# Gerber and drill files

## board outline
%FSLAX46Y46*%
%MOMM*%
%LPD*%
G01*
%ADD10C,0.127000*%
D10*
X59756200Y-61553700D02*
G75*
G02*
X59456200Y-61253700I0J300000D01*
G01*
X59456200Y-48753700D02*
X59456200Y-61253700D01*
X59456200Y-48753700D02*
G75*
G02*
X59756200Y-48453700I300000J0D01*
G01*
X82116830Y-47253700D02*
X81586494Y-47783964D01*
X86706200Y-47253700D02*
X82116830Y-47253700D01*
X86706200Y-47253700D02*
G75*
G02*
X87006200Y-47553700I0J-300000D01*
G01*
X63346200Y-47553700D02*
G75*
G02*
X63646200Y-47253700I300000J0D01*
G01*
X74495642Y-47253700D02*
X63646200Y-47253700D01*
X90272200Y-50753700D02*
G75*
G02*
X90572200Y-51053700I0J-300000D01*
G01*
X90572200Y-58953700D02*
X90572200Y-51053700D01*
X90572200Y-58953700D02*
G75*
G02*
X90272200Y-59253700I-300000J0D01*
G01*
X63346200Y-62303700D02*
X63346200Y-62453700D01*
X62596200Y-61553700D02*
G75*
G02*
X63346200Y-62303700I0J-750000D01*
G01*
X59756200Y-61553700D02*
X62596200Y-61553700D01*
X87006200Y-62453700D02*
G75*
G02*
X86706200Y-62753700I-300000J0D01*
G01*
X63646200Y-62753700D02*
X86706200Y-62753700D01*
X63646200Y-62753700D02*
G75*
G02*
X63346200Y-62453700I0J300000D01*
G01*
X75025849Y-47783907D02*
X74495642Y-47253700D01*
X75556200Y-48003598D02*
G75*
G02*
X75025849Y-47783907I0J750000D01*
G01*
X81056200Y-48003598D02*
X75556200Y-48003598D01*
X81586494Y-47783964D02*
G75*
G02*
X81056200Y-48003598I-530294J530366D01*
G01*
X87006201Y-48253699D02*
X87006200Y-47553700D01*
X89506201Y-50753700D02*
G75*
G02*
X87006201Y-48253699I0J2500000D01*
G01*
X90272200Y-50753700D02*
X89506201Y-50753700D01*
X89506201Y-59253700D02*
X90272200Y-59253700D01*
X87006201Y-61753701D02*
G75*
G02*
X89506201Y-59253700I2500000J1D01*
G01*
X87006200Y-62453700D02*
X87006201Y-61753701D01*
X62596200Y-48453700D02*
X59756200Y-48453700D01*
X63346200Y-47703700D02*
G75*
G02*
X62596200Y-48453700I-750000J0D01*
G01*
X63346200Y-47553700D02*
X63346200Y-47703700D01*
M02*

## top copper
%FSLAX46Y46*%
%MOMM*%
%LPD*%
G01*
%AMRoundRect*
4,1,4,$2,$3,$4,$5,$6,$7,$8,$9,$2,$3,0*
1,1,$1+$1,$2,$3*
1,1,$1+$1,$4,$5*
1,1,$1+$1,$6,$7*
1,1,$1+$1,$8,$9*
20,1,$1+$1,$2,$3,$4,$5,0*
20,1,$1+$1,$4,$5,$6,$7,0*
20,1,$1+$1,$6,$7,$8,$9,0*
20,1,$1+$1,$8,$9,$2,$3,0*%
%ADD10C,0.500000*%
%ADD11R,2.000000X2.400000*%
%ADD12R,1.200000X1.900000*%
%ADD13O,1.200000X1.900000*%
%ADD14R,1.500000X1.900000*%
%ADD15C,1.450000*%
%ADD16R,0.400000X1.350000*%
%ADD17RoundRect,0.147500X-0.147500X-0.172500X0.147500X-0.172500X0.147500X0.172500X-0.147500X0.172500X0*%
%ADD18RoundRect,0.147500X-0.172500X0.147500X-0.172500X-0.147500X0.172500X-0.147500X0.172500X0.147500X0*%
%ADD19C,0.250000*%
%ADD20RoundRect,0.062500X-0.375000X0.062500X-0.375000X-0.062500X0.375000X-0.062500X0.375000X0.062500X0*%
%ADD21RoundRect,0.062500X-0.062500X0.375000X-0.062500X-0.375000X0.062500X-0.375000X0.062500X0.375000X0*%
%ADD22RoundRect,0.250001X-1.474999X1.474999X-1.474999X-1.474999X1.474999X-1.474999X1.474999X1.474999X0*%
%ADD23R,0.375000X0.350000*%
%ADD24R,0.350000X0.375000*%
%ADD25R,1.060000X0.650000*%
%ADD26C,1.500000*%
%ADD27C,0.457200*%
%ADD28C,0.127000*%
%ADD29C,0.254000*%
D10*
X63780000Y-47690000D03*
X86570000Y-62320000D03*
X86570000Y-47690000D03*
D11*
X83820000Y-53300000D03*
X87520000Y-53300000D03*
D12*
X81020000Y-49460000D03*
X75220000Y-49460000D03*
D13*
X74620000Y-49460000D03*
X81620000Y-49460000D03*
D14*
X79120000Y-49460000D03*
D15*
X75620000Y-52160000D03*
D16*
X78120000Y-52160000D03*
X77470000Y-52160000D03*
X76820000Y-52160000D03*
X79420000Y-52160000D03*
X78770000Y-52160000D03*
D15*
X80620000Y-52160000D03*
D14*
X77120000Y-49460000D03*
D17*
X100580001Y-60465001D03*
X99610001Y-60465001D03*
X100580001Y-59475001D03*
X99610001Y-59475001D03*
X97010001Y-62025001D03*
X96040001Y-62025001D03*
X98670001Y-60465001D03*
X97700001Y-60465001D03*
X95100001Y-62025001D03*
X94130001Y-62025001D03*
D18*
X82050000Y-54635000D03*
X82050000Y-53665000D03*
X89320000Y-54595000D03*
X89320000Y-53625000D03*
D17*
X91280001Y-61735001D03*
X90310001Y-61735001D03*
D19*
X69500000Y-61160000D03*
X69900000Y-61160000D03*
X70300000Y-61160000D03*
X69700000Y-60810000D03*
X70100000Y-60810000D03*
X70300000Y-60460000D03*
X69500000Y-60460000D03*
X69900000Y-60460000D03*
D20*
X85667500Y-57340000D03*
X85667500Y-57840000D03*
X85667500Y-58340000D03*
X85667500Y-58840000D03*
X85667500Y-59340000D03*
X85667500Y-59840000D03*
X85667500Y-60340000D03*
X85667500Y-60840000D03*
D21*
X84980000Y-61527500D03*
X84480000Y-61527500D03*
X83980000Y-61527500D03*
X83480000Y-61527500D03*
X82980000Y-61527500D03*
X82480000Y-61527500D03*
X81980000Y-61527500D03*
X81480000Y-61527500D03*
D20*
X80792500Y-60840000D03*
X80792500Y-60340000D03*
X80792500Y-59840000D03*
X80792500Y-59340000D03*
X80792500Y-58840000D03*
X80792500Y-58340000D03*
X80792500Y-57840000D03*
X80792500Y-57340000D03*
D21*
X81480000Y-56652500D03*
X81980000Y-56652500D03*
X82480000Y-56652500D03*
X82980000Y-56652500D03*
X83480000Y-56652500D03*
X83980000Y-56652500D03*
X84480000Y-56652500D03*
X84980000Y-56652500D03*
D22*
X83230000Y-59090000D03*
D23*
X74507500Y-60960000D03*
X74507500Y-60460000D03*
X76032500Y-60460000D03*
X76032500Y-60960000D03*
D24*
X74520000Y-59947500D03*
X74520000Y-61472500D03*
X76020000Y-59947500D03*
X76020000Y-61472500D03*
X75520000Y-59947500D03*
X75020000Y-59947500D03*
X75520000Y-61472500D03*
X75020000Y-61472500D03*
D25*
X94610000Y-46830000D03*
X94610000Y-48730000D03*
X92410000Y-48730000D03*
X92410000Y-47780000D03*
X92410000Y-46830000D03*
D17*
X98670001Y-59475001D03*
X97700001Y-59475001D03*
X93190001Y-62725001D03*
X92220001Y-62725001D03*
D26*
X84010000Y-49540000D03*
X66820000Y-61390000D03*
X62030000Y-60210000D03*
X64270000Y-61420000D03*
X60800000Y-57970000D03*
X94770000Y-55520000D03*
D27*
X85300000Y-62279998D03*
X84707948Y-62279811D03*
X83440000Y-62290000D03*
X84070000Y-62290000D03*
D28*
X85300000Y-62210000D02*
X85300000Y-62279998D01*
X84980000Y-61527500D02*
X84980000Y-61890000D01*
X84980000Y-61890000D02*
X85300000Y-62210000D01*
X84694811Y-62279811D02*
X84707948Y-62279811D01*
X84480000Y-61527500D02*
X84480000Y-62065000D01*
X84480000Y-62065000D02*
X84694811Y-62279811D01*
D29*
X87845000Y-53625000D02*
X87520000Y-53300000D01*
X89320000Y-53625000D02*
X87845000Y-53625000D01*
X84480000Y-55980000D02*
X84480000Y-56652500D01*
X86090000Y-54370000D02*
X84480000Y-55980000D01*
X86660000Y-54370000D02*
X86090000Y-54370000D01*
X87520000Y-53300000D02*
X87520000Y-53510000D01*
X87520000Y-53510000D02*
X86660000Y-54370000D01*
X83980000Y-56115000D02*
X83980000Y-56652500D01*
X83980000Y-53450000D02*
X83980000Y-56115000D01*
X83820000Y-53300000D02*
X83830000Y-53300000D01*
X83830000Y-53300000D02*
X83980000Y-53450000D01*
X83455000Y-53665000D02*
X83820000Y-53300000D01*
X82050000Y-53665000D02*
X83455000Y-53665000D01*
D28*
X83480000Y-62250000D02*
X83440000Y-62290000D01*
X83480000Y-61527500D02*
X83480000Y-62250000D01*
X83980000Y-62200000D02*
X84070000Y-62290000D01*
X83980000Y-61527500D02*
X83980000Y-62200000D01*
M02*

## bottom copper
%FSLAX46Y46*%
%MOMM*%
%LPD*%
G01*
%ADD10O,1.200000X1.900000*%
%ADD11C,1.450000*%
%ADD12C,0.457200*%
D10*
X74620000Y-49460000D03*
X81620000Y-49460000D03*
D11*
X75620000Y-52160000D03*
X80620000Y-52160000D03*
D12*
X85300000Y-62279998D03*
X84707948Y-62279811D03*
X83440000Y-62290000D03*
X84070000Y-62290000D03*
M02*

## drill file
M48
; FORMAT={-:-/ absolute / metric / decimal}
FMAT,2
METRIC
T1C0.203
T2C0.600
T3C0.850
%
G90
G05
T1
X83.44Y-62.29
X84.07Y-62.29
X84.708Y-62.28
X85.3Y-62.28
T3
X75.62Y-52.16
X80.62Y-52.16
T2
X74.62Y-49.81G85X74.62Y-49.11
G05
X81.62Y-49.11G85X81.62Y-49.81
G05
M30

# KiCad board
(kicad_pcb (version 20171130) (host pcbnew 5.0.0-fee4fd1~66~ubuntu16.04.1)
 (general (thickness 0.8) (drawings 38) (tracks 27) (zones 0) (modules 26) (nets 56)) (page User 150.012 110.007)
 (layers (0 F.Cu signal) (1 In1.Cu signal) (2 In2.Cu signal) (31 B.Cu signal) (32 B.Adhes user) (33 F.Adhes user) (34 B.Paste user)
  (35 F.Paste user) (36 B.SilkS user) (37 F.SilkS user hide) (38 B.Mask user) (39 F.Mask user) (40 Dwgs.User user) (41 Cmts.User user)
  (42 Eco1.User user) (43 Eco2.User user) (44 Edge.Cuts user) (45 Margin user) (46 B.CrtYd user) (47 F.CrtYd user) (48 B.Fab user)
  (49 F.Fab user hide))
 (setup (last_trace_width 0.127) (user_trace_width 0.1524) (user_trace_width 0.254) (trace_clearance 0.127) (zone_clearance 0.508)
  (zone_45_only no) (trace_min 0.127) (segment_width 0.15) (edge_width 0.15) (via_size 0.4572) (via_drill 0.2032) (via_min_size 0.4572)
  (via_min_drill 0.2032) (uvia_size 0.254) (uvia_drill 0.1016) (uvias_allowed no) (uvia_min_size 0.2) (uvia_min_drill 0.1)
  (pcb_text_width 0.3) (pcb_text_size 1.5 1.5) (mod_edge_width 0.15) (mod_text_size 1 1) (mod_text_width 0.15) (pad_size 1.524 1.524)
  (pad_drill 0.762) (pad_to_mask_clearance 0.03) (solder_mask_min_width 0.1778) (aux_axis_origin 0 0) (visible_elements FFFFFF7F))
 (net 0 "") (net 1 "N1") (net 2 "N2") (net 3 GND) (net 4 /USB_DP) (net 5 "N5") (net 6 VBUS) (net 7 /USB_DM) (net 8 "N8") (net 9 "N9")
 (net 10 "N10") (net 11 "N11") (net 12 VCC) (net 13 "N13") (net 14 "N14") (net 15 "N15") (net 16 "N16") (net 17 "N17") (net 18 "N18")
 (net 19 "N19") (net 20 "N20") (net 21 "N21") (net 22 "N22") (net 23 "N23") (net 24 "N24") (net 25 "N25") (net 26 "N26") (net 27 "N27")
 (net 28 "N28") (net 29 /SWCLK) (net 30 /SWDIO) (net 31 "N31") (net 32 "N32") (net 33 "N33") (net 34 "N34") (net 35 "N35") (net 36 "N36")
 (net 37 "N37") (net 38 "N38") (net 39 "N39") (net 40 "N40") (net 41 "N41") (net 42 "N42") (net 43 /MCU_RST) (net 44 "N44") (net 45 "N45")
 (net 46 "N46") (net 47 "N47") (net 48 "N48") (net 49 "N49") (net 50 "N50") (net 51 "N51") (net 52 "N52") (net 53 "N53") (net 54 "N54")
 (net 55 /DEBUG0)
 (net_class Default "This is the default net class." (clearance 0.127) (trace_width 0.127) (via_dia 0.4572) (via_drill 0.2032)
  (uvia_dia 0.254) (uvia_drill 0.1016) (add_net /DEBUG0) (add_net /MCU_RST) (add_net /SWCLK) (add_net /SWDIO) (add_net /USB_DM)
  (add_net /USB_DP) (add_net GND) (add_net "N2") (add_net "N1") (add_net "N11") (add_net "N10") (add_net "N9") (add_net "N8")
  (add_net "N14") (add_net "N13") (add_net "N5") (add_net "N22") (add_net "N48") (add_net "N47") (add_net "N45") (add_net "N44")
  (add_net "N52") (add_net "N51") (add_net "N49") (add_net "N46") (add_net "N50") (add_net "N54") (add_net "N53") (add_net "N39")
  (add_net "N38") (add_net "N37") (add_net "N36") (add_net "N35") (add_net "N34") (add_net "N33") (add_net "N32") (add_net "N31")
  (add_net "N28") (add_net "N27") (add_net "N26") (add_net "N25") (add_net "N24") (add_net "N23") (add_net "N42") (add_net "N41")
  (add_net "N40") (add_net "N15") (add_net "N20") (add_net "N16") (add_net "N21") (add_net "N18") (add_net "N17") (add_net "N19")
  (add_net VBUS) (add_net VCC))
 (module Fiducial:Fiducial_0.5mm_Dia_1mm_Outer (layer F.Cu) (at 63.78 47.69)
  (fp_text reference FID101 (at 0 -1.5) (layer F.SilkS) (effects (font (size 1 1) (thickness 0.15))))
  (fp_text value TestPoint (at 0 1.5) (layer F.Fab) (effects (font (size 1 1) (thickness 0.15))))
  (pad ~ smd circle (at 0 0) (size 0.5 0.5) (layers F.Cu F.Mask) (solder_mask_margin 0.25) (clearance 0.25)))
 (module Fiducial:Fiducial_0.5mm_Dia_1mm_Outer (layer F.Cu) (at 86.57 62.32)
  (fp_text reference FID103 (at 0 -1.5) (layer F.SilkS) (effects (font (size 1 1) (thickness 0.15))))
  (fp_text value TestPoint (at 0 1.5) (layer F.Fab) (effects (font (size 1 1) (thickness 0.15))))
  (pad ~ smd circle (at 0 0) (size 0.5 0.5) (layers F.Cu F.Mask) (solder_mask_margin 0.25) (clearance 0.25)))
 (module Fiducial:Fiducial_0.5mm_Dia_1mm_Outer (layer F.Cu) (at 86.57 47.69)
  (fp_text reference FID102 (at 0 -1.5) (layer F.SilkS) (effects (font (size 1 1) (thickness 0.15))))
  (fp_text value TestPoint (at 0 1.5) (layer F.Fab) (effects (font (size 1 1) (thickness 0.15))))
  (pad ~ smd circle (at 0 0) (size 0.5 0.5) (layers F.Cu F.Mask) (solder_mask_margin 0.25) (clearance 0.25)))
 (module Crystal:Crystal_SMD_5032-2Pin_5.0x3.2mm (layer F.Cu) (at 85.67 53.3 180)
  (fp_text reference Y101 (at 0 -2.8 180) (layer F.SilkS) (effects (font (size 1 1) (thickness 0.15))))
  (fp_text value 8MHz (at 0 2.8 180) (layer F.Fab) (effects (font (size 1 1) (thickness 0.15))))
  (pad 2 smd rect (at 1.85 0 180) (size 2 2.4) (layers F.Cu F.Paste F.Mask) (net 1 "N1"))
  (pad 1 smd rect (at -1.85 0 180) (size 2 2.4) (layers F.Cu F.Paste F.Mask) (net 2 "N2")))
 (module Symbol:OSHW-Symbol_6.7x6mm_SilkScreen (layer F.Cu) (at 67.84 53.39 270)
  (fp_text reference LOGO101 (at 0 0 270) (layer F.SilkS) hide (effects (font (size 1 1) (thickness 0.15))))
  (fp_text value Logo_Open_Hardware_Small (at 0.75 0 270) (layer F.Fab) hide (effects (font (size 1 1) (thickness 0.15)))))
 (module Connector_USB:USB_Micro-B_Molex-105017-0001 (layer F.Cu) (at 78.12 50.6975 180)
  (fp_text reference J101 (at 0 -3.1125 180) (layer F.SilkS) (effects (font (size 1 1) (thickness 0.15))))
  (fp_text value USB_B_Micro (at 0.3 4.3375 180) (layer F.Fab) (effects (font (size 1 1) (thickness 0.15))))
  (pad 6 smd rect (at -2.9 1.2375 180) (size 1.2 1.9) (layers F.Cu F.Mask) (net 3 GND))
  (pad 6 smd rect (at 2.9 1.2375 180) (size 1.2 1.9) (layers F.Cu F.Mask) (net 3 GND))
  (pad 6 thru_hole oval (at 3.5 1.2375 180) (size 1.2 1.9) (drill oval 0.6 1.3) (layers *.Cu *.Mask) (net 3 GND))
  (pad 6 thru_hole oval (at -3.5 1.2375) (size 1.2 1.9) (drill oval 0.6 1.3) (layers *.Cu *.Mask) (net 3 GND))
  (pad 6 smd rect (at -1 1.2375 180) (size 1.5 1.9) (layers F.Cu F.Paste F.Mask) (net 3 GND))
  (pad 6 thru_hole circle (at 2.5 -1.4625 180) (size 1.45 1.45) (drill 0.85) (layers *.Cu *.Mask) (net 3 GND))
  (pad 3 smd rect (at 0 -1.4625 180) (size 0.4 1.35) (layers F.Cu F.Paste F.Mask) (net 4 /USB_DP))
  (pad 4 smd rect (at 0.65 -1.4625 180) (size 0.4 1.35) (layers F.Cu F.Paste F.Mask) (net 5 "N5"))
  (pad 5 smd rect (at 1.3 -1.4625 180) (size 0.4 1.35) (layers F.Cu F.Paste F.Mask) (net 3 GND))
  (pad 1 smd rect (at -1.3 -1.4625 180) (size 0.4 1.35) (layers F.Cu F.Paste F.Mask) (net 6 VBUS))
  (pad 2 smd rect (at -0.65 -1.4625 180) (size 0.4 1.35) (layers F.Cu F.Paste F.Mask) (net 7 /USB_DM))
  (pad 6 thru_hole circle (at -2.5 -1.4625 180) (size 1.45 1.45) (drill 0.85) (layers *.Cu *.Mask) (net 3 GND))
  (pad 6 smd rect (at 1 1.2375 180) (size 1.5 1.9) (layers F.Cu F.Paste F.Mask) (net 3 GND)))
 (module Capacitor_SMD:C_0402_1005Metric (layer F.Cu) (at 100.095001 60.465001)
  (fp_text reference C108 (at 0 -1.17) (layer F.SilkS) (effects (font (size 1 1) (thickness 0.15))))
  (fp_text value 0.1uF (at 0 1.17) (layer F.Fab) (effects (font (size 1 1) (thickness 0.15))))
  (pad 2 smd roundrect (at 0.485 0) (size 0.59 0.64) (layers F.Cu F.Paste F.Mask) (roundrect_rratio 0.25) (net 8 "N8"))
  (pad 1 smd roundrect (at -0.485 0) (size 0.59 0.64) (layers F.Cu F.Paste F.Mask) (roundrect_rratio 0.25) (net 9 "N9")))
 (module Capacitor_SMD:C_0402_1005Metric (layer F.Cu) (at 100.095001 59.475001)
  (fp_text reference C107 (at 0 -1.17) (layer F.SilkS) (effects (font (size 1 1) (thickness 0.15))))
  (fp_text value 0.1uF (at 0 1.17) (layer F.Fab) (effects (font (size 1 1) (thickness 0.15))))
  (pad 2 smd roundrect (at 0.485 0) (size 0.59 0.64) (layers F.Cu F.Paste F.Mask) (roundrect_rratio 0.25) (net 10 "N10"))
  (pad 1 smd roundrect (at -0.485 0) (size 0.59 0.64) (layers F.Cu F.Paste F.Mask) (roundrect_rratio 0.25) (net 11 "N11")))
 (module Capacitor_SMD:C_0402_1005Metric (layer F.Cu) (at 96.525001 62.025001)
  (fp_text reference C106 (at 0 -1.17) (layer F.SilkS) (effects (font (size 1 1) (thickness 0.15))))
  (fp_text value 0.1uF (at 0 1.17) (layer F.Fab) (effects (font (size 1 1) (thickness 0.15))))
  (pad 2 smd roundrect (at 0.485 0) (size 0.59 0.64) (layers F.Cu F.Paste F.Mask) (roundrect_rratio 0.25) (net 3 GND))
  (pad 1 smd roundrect (at -0.485 0) (size 0.59 0.64) (layers F.Cu F.Paste F.Mask) (roundrect_rratio 0.25) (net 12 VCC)))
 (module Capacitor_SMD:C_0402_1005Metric (layer F.Cu) (at 98.185001 60.465001)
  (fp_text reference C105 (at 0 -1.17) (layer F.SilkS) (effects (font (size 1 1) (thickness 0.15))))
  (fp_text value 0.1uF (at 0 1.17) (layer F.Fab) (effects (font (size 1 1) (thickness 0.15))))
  (pad 2 smd roundrect (at 0.485 0) (size 0.59 0.64) (layers F.Cu F.Paste F.Mask) (roundrect_rratio 0.25) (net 3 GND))
  (pad 1 smd roundrect (at -0.485 0) (size 0.59 0.64) (layers F.Cu F.Paste F.Mask) (roundrect_rratio 0.25) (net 12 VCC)))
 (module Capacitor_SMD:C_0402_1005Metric (layer F.Cu) (at 94.615001 62.025001)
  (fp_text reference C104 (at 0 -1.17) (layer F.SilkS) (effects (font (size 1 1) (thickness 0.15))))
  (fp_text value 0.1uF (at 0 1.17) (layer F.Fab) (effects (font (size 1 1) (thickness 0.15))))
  (pad 2 smd roundrect (at 0.485 0) (size 0.59 0.64) (layers F.Cu F.Paste F.Mask) (roundrect_rratio 0.25) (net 3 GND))
  (pad 1 smd roundrect (at -0.485 0) (size 0.59 0.64) (layers F.Cu F.Paste F.Mask) (roundrect_rratio 0.25) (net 12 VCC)))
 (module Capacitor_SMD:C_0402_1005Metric (layer F.Cu) (at 82.05 54.15 270)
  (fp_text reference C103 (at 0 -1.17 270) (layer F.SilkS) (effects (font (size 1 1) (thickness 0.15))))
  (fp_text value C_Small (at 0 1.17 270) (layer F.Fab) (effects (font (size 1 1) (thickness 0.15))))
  (pad 2 smd roundrect (at 0.485 0 270) (size 0.59 0.64) (layers F.Cu F.Paste F.Mask) (roundrect_rratio 0.25) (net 3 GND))
  (pad 1 smd roundrect (at -0.485 0 270) (size 0.59 0.64) (layers F.Cu F.Paste F.Mask) (roundrect_rratio 0.25) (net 1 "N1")))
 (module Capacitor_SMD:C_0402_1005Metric (layer F.Cu) (at 89.32 54.11 270)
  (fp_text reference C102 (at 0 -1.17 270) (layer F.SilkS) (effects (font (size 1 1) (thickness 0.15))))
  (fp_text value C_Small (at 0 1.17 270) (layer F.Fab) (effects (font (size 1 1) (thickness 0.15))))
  (pad 2 smd roundrect (at 0.485 0 270) (size 0.59 0.64) (layers F.Cu F.Paste F.Mask) (roundrect_rratio 0.25) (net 3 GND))
  (pad 1 smd roundrect (at -0.485 0 270) (size 0.59 0.64) (layers F.Cu F.Paste F.Mask) (roundrect_rratio 0.25) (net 2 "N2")))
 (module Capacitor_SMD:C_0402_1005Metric (layer F.Cu) (at 90.795001 61.735001)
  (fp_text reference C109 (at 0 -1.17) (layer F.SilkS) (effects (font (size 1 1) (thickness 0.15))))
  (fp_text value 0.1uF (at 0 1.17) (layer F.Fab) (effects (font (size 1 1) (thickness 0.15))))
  (pad 2 smd roundrect (at 0.485 0) (size 0.59 0.64) (layers F.Cu F.Paste F.Mask) (roundrect_rratio 0.25) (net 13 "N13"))
  (pad 1 smd roundrect (at -0.485 0) (size 0.59 0.64) (layers F.Cu F.Paste F.Mask) (roundrect_rratio 0.25) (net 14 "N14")))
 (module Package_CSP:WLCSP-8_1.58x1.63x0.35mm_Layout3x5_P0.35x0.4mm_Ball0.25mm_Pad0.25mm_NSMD (layer F.Cu) (at 69.9 60.81 90)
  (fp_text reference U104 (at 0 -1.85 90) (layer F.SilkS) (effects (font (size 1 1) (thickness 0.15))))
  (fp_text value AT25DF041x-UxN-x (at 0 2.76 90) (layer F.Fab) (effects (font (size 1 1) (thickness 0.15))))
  (pad A1 smd circle (at -0.35 -0.4 90) (size 0.25 0.25) (layers F.Cu F.Paste F.Mask) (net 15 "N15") (solder_mask_margin 0.03))
  (pad C1 smd circle (at -0.35 0 90) (size 0.25 0.25) (layers F.Cu F.Paste F.Mask) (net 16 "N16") (solder_mask_margin 0.03))
  (pad E1 smd circle (at -0.35 0.4 90) (size 0.25 0.25) (layers F.Cu F.Paste F.Mask) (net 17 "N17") (solder_mask_margin 0.03))
  (pad B2 smd circle (at 0 -0.2 90) (size 0.25 0.25) (layers F.Cu F.Paste F.Mask) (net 3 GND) (solder_mask_margin 0.03))
  (pad D2 smd circle (at 0 0.2 90) (size 0.25 0.25) (layers F.Cu F.Paste F.Mask) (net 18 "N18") (solder_mask_margin 0.03))
  (pad E3 smd circle (at 0.35 0.4 90) (size 0.25 0.25) (layers F.Cu F.Paste F.Mask) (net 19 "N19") (solder_mask_margin 0.03))
  (pad A3 smd circle (at 0.35 -0.4 90) (size 0.25 0.25) (layers F.Cu F.Paste F.Mask) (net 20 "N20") (solder_mask_margin 0.03))
  (pad C3 smd circle (at 0.35 0 90) (size 0.25 0.25) (layers F.Cu F.Paste F.Mask) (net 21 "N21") (solder_mask_margin 0.03)))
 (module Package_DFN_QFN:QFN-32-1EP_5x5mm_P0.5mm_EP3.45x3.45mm (layer F.Cu) (at 83.23 59.09 270)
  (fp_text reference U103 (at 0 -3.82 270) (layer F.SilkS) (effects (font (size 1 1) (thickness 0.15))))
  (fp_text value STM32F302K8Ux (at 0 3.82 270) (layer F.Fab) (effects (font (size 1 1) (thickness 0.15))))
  (pad 32 smd roundrect (at -1.75 -2.4375 270) (size 0.25 0.875) (layers F.Cu F.Paste F.Mask) (roundrect_rratio 0.25) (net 3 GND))
  (pad 31 smd roundrect (at -1.25 -2.4375 270) (size 0.25 0.875) (layers F.Cu F.Paste F.Mask) (roundrect_rratio 0.25) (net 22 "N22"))
  (pad 30 smd roundrect (at -0.75 -2.4375 270) (size 0.25 0.875) (layers F.Cu F.Paste F.Mask) (roundrect_rratio 0.25) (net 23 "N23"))
  (pad 29 smd roundrect (at -0.25 -2.4375 270) (size 0.25 0.875) (layers F.Cu F.Paste F.Mask) (roundrect_rratio 0.25) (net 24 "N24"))
  (pad 28 smd roundrect (at 0.25 -2.4375 270) (size 0.25 0.875) (layers F.Cu F.Paste F.Mask) (roundrect_rratio 0.25) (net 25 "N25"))
  (pad 27 smd roundrect (at 0.75 -2.4375 270) (size 0.25 0.875) (layers F.Cu F.Paste F.Mask) (roundrect_rratio 0.25) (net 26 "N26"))
  (pad 26 smd roundrect (at 1.25 -2.4375 270) (size 0.25 0.875) (layers F.Cu F.Paste F.Mask) (roundrect_rratio 0.25) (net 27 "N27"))
  (pad 25 smd roundrect (at 1.75 -2.4375 270) (size 0.25 0.875) (layers F.Cu F.Paste F.Mask) (roundrect_rratio 0.25) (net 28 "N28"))
  (pad 24 smd roundrect (at 2.4375 -1.75 270) (size 0.875 0.25) (layers F.Cu F.Paste F.Mask) (roundrect_rratio 0.25) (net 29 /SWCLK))
  (pad 23 smd roundrect (at 2.4375 -1.25 270) (size 0.875 0.25) (layers F.Cu F.Paste F.Mask) (roundrect_rratio 0.25) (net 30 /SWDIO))
  (pad 22 smd roundrect (at 2.4375 -0.75 270) (size 0.875 0.25) (layers F.Cu F.Paste F.Mask) (roundrect_rratio 0.25) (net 4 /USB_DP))
  (pad 21 smd roundrect (at 2.4375 -0.25 270) (size 0.875 0.25) (layers F.Cu F.Paste F.Mask) (roundrect_rratio 0.25) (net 7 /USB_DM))
  (pad 20 smd roundrect (at 2.4375 0.25 270) (size 0.875 0.25) (layers F.Cu F.Paste F.Mask) (roundrect_rratio 0.25) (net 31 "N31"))
  (pad 19 smd roundrect (at 2.4375 0.75 270) (size 0.875 0.25) (layers F.Cu F.Paste F.Mask) (roundrect_rratio 0.25) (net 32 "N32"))
  (pad 18 smd roundrect (at 2.4375 1.25 270) (size 0.875 0.25) (layers F.Cu F.Paste F.Mask) (roundrect_rratio 0.25) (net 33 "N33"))
  (pad 17 smd roundrect (at 2.4375 1.75 270) (size 0.875 0.25) (layers F.Cu F.Paste F.Mask) (roundrect_rratio 0.25) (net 12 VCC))
  (pad 16 smd roundrect (at 1.75 2.4375 270) (size 0.25 0.875) (layers F.Cu F.Paste F.Mask) (roundrect_rratio 0.25) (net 3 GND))
  (pad 15 smd roundrect (at 1.25 2.4375 270) (size 0.25 0.875) (layers F.Cu F.Paste F.Mask) (roundrect_rratio 0.25) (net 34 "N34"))
  (pad 14 smd roundrect (at 0.75 2.4375 270) (size 0.25 0.875) (layers F.Cu F.Paste F.Mask) (roundrect_rratio 0.25) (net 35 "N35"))
  (pad 13 smd roundrect (at 0.25 2.4375 270) (size 0.25 0.875) (layers F.Cu F.Paste F.Mask) (roundrect_rratio 0.25) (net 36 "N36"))
  (pad 12 smd roundrect (at -0.25 2.4375 270) (size 0.25 0.875) (layers F.Cu F.Paste F.Mask) (roundrect_rratio 0.25) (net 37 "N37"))
  (pad 11 smd roundrect (at -0.75 2.4375 270) (size 0.25 0.875) (layers F.Cu F.Paste F.Mask) (roundrect_rratio 0.25) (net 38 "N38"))
  (pad 10 smd roundrect (at -1.25 2.4375 270) (size 0.25 0.875) (layers F.Cu F.Paste F.Mask) (roundrect_rratio 0.25) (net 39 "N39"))
  (pad 9 smd roundrect (at -1.75 2.4375 270) (size 0.25 0.875) (layers F.Cu F.Paste F.Mask) (roundrect_rratio 0.25) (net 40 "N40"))
  (pad 8 smd roundrect (at -2.4375 1.75 270) (size 0.875 0.25) (layers F.Cu F.Paste F.Mask) (roundrect_rratio 0.25) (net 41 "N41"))
  (pad 7 smd roundrect (at -2.4375 1.25 270) (size 0.875 0.25) (layers F.Cu F.Paste F.Mask) (roundrect_rratio 0.25) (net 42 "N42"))
  (pad 6 smd roundrect (at -2.4375 0.75 270) (size 0.875 0.25) (layers F.Cu F.Paste F.Mask) (roundrect_rratio 0.25) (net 3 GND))
  (pad 5 smd roundrect (at -2.4375 0.25 270) (size 0.875 0.25) (layers F.Cu F.Paste F.Mask) (roundrect_rratio 0.25) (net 12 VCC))
  (pad 4 smd roundrect (at -2.4375 -0.25 270) (size 0.875 0.25) (layers F.Cu F.Paste F.Mask) (roundrect_rratio 0.25) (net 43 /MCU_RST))
  (pad 3 smd roundrect (at -2.4375 -0.75 270) (size 0.875 0.25) (layers F.Cu F.Paste F.Mask) (roundrect_rratio 0.25) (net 1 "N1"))
  (pad 2 smd roundrect (at -2.4375 -1.25 270) (size 0.875 0.25) (layers F.Cu F.Paste F.Mask) (roundrect_rratio 0.25) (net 2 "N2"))
  (pad 1 smd roundrect (at -2.4375 -1.75 270) (size 0.875 0.25) (layers F.Cu F.Paste F.Mask) (roundrect_rratio 0.25) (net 12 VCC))
  (pad "" smd roundrect (at 1.15 1.15 270) (size 0.93 0.93) (layers F.Paste) (roundrect_rratio 0.25))
  (pad "" smd roundrect (at 1.15 0 270) (size 0.93 0.93) (layers F.Paste) (roundrect_rratio 0.25))
  (pad "" smd roundrect (at 1.15 -1.15 270) (size 0.93 0.93) (layers F.Paste) (roundrect_rratio 0.25))
  (pad "" smd roundrect (at 0 1.15 270) (size 0.93 0.93) (layers F.Paste) (roundrect_rratio 0.25))
  (pad "" smd roundrect (at 0 0 270) (size 0.93 0.93) (layers F.Paste) (roundrect_rratio 0.25))
  (pad "" smd roundrect (at 0 -1.15 270) (size 0.93 0.93) (layers F.Paste) (roundrect_rratio 0.25))
  (pad "" smd roundrect (at -1.15 1.15 270) (size 0.93 0.93) (layers F.Paste) (roundrect_rratio 0.25))
  (pad "" smd roundrect (at -1.15 0 270) (size 0.93 0.93) (layers F.Paste) (roundrect_rratio 0.25))
  (pad "" smd roundrect (at -1.15 -1.15 270) (size 0.93 0.93) (layers F.Paste) (roundrect_rratio 0.25))
  (pad 33 smd roundrect (at 0 0 270) (size 3.45 3.45) (layers F.Cu F.Mask) (roundrect_rratio 0.072464) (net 3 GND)))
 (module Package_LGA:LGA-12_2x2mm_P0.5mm (layer F.Cu) (at 75.27 60.71 90)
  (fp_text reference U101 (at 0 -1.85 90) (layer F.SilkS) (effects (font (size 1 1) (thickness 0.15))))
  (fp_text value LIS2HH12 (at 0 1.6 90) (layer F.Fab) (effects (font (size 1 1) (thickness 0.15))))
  (pad 12 smd rect (at -0.25 -0.7625 180) (size 0.375 0.35) (layers F.Cu F.Paste F.Mask) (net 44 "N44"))
  (pad 11 smd rect (at 0.25 -0.7625 180) (size 0.375 0.35) (layers F.Cu F.Paste F.Mask) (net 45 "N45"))
  (pad 6 smd rect (at 0.25 0.7625 180) (size 0.375 0.35) (layers F.Cu F.Paste F.Mask) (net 3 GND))
  (pad 5 smd rect (at -0.25 0.7625 180) (size 0.375 0.35) (layers F.Cu F.Paste F.Mask) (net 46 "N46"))
  (pad 10 smd rect (at 0.7625 -0.75 90) (size 0.375 0.35) (layers F.Cu F.Paste F.Mask) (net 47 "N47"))
  (pad 1 smd rect (at -0.7625 -0.75 90) (size 0.375 0.35) (layers F.Cu F.Paste F.Mask) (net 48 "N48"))
  (pad 7 smd rect (at 0.7625 0.75 90) (size 0.375 0.35) (layers F.Cu F.Paste F.Mask) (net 3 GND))
  (pad 4 smd rect (at -0.7625 0.75 90) (size 0.375 0.35) (layers F.Cu F.Paste F.Mask) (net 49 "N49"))
  (pad 8 smd rect (at 0.7625 0.25 90) (size 0.375 0.35) (layers F.Cu F.Paste F.Mask) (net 3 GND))
  (pad 9 smd rect (at 0.7625 -0.25 90) (size 0.375 0.35) (layers F.Cu F.Paste F.Mask) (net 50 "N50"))
  (pad 3 smd rect (at -0.7625 0.25 90) (size 0.375 0.35) (layers F.Cu F.Paste F.Mask) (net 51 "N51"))
  (pad 2 smd rect (at -0.7625 -0.25 90) (size 0.375 0.35) (layers F.Cu F.Paste F.Mask) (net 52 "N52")))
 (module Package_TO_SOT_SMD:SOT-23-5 (layer F.Cu) (at 93.51 47.78)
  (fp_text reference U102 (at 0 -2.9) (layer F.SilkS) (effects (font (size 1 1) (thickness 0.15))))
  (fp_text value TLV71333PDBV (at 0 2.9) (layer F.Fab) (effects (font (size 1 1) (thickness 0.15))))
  (pad 5 smd rect (at 1.1 -0.95) (size 1.06 0.65) (layers F.Cu F.Paste F.Mask) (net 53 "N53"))
  (pad 4 smd rect (at 1.1 0.95) (size 1.06 0.65) (layers F.Cu F.Paste F.Mask) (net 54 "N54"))
  (pad 3 smd rect (at -1.1 0.95) (size 1.06 0.65) (layers F.Cu F.Paste F.Mask) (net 6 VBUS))
  (pad 2 smd rect (at -1.1 0) (size 1.06 0.65) (layers F.Cu F.Paste F.Mask) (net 3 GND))
  (pad 1 smd rect (at -1.1 -0.95) (size 1.06 0.65) (layers F.Cu F.Paste F.Mask) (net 6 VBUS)))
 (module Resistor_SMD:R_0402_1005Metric (layer F.Cu) (at 98.185001 59.475001)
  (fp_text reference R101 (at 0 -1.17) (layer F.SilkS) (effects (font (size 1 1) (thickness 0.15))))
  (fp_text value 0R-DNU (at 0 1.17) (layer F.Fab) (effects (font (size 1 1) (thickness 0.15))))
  (pad 2 smd roundrect (at 0.485 0) (size 0.59 0.64) (layers F.Cu F.Paste F.Mask) (roundrect_rratio 0.25) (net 22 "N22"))
  (pad 1 smd roundrect (at -0.485 0) (size 0.59 0.64) (layers F.Cu F.Paste F.Mask) (roundrect_rratio 0.25) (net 12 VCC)))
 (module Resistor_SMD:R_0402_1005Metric (layer F.Cu) (at 92.705001 62.725001)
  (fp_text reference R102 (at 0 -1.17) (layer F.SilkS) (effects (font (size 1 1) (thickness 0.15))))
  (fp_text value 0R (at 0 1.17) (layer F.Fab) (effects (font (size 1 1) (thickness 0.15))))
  (pad 2 smd roundrect (at 0.485 0) (size 0.59 0.64) (layers F.Cu F.Paste F.Mask) (roundrect_rratio 0.25) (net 3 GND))
  (pad 1 smd roundrect (at -0.485 0) (size 0.59 0.64) (layers F.Cu F.Paste F.Mask) (roundrect_rratio 0.25) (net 22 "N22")))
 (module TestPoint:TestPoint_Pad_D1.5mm (layer F.Cu) (at 84.01 49.54)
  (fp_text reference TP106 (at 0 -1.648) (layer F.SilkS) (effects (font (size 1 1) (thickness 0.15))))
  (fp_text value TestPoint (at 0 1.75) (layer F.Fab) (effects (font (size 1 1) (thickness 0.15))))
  (pad 1 smd circle (at 0 0) (size 1.5 1.5) (layers F.Cu F.Mask) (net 3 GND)))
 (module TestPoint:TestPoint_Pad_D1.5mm (layer F.Cu) (at 66.82 61.39)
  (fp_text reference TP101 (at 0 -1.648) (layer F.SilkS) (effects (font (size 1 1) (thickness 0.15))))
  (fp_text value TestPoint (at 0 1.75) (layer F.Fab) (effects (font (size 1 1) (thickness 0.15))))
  (pad 1 smd circle (at 0 0) (size 1.5 1.5) (layers F.Cu F.Mask) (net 43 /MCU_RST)))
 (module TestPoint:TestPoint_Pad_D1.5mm (layer F.Cu) (at 62.03 60.21)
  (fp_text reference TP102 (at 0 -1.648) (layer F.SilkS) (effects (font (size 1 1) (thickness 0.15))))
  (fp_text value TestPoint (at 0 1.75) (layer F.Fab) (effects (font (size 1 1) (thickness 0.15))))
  (pad 1 smd circle (at 0 0) (size 1.5 1.5) (layers F.Cu F.Mask) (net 30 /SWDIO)))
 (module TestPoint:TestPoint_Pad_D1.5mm (layer F.Cu) (at 64.27 61.42)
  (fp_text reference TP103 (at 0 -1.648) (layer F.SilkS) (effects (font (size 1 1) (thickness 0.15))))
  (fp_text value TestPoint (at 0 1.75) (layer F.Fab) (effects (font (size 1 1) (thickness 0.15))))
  (pad 1 smd circle (at 0 0) (size 1.5 1.5) (layers F.Cu F.Mask) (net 29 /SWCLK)))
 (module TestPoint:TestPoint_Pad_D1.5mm (layer F.Cu) (at 60.8 57.97)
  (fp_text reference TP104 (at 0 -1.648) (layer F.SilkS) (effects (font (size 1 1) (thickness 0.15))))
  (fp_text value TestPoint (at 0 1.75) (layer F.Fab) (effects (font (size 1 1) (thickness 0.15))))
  (pad 1 smd circle (at 0 0) (size 1.5 1.5) (layers F.Cu F.Mask) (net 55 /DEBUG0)))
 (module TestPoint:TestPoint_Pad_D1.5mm (layer F.Cu) (at 94.77 55.52)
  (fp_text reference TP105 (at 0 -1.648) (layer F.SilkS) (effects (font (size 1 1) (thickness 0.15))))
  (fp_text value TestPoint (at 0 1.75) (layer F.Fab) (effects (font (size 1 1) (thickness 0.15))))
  (pad 1 smd circle (at 0 0) (size 1.5 1.5) (layers F.Cu F.Mask) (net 12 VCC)))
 (gr_arc (start 59.7562 61.2537) (end 59.4562 61.2537) (angle -90.00000085) (layer Edge.Cuts) (width 0.127))
 (gr_line (start 59.4562 48.7537) (end 59.4562 61.2537) (layer Edge.Cuts) (width 0.127))
 (gr_arc (start 59.7562 48.7537) (end 59.7562 48.4537) (angle -89.99999915) (layer Edge.Cuts) (width 0.127))
 (gr_line (start 82.11683 47.2537) (end 81.586494 47.783964) (layer Edge.Cuts) (width 0.127))
 (gr_line (start 86.7062 47.2537) (end 82.11683 47.2537) (layer Edge.Cuts) (width 0.127))
 (gr_arc (start 86.7062 47.5537) (end 87.0062 47.5537) (angle -90) (layer Edge.Cuts) (width 0.127))
 (gr_arc (start 63.6462 47.5537) (end 63.6462 47.2537) (angle -90) (layer Edge.Cuts) (width 0.127))
 (gr_line (start 74.495642 47.2537) (end 63.6462 47.2537) (layer Edge.Cuts) (width 0.127))
 (gr_arc (start 90.2722 51.0537) (end 90.5722 51.0537) (angle -90) (layer Edge.Cuts) (width 0.127))
 (gr_line (start 90.5722 58.9537) (end 90.5722 51.0537) (layer Edge.Cuts) (width 0.127))
 (gr_arc (start 90.2722 58.9537) (end 90.2722 59.2537) (angle -90) (layer Edge.Cuts) (width 0.127))
 (gr_line (start 63.3462 62.3037) (end 63.3462 62.4537) (layer Edge.Cuts) (width 0.127))
 (gr_arc (start 62.5962 62.3037) (end 63.3462 62.3037) (angle -90) (layer Edge.Cuts) (width 0.127))
 (gr_line (start 59.7562 61.5537) (end 62.5962 61.5537) (layer Edge.Cuts) (width 0.127))
 (gr_arc (start 86.7062 62.4537) (end 86.7062 62.7537) (angle -89.99999944) (layer Edge.Cuts) (width 0.127))
 (gr_line (start 63.6462 62.7537) (end 86.7062 62.7537) (layer Edge.Cuts) (width 0.127))
 (gr_arc (start 63.6462 62.4537) (end 63.3462 62.4537) (angle -90.00000056) (layer Edge.Cuts) (width 0.127))
 (gr_line (start 75.025849 47.783907) (end 74.495642 47.2537) (layer Edge.Cuts) (width 0.127))
 (gr_arc (start 75.5562 47.253598) (end 75.025849 47.783907) (angle -45.00225503) (layer Edge.Cuts) (width 0.127))
 (gr_line (start 81.0562 48.003598) (end 75.5562 48.003598) (layer Edge.Cuts) (width 0.127))
 (gr_arc (start 81.0562 47.253598) (end 81.0562 48.003598) (angle -44.99610213) (layer Edge.Cuts) (width 0.127))
 (gr_line (start 87.006201 48.253699) (end 87.0062 47.5537) (layer Edge.Cuts) (width 0.127))
 (gr_arc (start 89.506201 48.2537) (end 87.006201 48.253699) (angle -90.00002618) (layer Edge.Cuts) (width 0.127))
 (gr_line (start 90.2722 50.7537) (end 89.506201 50.7537) (layer Edge.Cuts) (width 0.127))
 (gr_line (start 89.506201 59.2537) (end 90.2722 59.2537) (layer Edge.Cuts) (width 0.127))
 (gr_arc (start 89.506201 61.7537) (end 89.506201 59.2537) (angle -90.00002618) (layer Edge.Cuts) (width 0.127))
 (gr_line (start 87.0062 62.4537) (end 87.006201 61.753701) (layer Edge.Cuts) (width 0.127))
 (gr_line (start 62.5962 48.4537) (end 59.7562 48.4537) (layer Edge.Cuts) (width 0.127))
 (gr_arc (start 62.5962 47.7037) (end 62.5962 48.4537) (angle -90) (layer Edge.Cuts) (width 0.127))
 (gr_line (start 63.3462 47.5537) (end 63.3462 47.7037) (layer Edge.Cuts) (width 0.127))
 (via (at 85.3 62.279998) (size 0.4572) (drill 0.2032) (layers F.Cu B.Cu) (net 29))
 (segment (start 85.3 62.21) (end 85.3 62.279998) (width 0.127) (layer F.Cu) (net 29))
 (segment (start 84.98 61.5275) (end 84.98 61.89) (width 0.127) (layer F.Cu) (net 29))
 (segment (start 84.98 61.89) (end 85.3 62.21) (width 0.127) (layer F.Cu) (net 29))
 (segment (start 84.694811 62.279811) (end 84.707948 62.279811) (width 0.127) (layer F.Cu) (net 30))
 (segment (start 84.48 61.5275) (end 84.48 62.065) (width 0.127) (layer F.Cu) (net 30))
 (segment (start 84.48 62.065) (end 84.694811 62.279811) (width 0.127) (layer F.Cu) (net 30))
 (via (at 84.707948 62.279811) (size 0.4572) (drill 0.2032) (layers F.Cu B.Cu) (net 30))
 (segment (start 87.845 53.625) (end 87.52 53.3) (width 0.254) (layer F.Cu) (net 2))
 (segment (start 89.32 53.625) (end 87.845 53.625) (width 0.254) (layer F.Cu) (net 2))
 (segment (start 84.48 55.98) (end 84.48 56.6525) (width 0.254) (layer F.Cu) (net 2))
 (segment (start 86.09 54.37) (end 84.48 55.98) (width 0.254) (layer F.Cu) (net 2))
 (segment (start 86.66 54.37) (end 86.09 54.37) (width 0.254) (layer F.Cu) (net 2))
 (segment (start 87.52 53.3) (end 87.52 53.51) (width 0.254) (layer F.Cu) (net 2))
 (segment (start 87.52 53.51) (end 86.66 54.37) (width 0.254) (layer F.Cu) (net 2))
 (segment (start 83.98 56.115) (end 83.98 56.6525) (width 0.254) (layer F.Cu) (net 1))
 (segment (start 83.98 53.45) (end 83.98 56.115) (width 0.254) (layer F.Cu) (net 1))
 (segment (start 83.82 53.3) (end 83.83 53.3) (width 0.254) (layer F.Cu) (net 1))
 (segment (start 83.83 53.3) (end 83.98 53.45) (width 0.254) (layer F.Cu) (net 1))
 (segment (start 83.455 53.665) (end 83.82 53.3) (width 0.254) (layer F.Cu) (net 1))
 (segment (start 82.05 53.665) (end 83.455 53.665) (width 0.254) (layer F.Cu) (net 1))
 (via (at 83.44 62.29) (size 0.4572) (drill 0.2032) (layers F.Cu B.Cu) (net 7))
 (segment (start 83.48 62.25) (end 83.44 62.29) (width 0.127) (layer F.Cu) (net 7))
 (segment (start 83.48 61.5275) (end 83.48 62.25) (width 0.127) (layer F.Cu) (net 7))
 (via (at 84.07 62.29) (size 0.4572) (drill 0.2032) (layers F.Cu B.Cu) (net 4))
 (segment (start 83.98 62.2) (end 84.07 62.29) (width 0.127) (layer F.Cu) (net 4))
 (segment (start 83.98 61.5275) (end 83.98 62.2) (width 0.127) (layer F.Cu) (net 4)))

